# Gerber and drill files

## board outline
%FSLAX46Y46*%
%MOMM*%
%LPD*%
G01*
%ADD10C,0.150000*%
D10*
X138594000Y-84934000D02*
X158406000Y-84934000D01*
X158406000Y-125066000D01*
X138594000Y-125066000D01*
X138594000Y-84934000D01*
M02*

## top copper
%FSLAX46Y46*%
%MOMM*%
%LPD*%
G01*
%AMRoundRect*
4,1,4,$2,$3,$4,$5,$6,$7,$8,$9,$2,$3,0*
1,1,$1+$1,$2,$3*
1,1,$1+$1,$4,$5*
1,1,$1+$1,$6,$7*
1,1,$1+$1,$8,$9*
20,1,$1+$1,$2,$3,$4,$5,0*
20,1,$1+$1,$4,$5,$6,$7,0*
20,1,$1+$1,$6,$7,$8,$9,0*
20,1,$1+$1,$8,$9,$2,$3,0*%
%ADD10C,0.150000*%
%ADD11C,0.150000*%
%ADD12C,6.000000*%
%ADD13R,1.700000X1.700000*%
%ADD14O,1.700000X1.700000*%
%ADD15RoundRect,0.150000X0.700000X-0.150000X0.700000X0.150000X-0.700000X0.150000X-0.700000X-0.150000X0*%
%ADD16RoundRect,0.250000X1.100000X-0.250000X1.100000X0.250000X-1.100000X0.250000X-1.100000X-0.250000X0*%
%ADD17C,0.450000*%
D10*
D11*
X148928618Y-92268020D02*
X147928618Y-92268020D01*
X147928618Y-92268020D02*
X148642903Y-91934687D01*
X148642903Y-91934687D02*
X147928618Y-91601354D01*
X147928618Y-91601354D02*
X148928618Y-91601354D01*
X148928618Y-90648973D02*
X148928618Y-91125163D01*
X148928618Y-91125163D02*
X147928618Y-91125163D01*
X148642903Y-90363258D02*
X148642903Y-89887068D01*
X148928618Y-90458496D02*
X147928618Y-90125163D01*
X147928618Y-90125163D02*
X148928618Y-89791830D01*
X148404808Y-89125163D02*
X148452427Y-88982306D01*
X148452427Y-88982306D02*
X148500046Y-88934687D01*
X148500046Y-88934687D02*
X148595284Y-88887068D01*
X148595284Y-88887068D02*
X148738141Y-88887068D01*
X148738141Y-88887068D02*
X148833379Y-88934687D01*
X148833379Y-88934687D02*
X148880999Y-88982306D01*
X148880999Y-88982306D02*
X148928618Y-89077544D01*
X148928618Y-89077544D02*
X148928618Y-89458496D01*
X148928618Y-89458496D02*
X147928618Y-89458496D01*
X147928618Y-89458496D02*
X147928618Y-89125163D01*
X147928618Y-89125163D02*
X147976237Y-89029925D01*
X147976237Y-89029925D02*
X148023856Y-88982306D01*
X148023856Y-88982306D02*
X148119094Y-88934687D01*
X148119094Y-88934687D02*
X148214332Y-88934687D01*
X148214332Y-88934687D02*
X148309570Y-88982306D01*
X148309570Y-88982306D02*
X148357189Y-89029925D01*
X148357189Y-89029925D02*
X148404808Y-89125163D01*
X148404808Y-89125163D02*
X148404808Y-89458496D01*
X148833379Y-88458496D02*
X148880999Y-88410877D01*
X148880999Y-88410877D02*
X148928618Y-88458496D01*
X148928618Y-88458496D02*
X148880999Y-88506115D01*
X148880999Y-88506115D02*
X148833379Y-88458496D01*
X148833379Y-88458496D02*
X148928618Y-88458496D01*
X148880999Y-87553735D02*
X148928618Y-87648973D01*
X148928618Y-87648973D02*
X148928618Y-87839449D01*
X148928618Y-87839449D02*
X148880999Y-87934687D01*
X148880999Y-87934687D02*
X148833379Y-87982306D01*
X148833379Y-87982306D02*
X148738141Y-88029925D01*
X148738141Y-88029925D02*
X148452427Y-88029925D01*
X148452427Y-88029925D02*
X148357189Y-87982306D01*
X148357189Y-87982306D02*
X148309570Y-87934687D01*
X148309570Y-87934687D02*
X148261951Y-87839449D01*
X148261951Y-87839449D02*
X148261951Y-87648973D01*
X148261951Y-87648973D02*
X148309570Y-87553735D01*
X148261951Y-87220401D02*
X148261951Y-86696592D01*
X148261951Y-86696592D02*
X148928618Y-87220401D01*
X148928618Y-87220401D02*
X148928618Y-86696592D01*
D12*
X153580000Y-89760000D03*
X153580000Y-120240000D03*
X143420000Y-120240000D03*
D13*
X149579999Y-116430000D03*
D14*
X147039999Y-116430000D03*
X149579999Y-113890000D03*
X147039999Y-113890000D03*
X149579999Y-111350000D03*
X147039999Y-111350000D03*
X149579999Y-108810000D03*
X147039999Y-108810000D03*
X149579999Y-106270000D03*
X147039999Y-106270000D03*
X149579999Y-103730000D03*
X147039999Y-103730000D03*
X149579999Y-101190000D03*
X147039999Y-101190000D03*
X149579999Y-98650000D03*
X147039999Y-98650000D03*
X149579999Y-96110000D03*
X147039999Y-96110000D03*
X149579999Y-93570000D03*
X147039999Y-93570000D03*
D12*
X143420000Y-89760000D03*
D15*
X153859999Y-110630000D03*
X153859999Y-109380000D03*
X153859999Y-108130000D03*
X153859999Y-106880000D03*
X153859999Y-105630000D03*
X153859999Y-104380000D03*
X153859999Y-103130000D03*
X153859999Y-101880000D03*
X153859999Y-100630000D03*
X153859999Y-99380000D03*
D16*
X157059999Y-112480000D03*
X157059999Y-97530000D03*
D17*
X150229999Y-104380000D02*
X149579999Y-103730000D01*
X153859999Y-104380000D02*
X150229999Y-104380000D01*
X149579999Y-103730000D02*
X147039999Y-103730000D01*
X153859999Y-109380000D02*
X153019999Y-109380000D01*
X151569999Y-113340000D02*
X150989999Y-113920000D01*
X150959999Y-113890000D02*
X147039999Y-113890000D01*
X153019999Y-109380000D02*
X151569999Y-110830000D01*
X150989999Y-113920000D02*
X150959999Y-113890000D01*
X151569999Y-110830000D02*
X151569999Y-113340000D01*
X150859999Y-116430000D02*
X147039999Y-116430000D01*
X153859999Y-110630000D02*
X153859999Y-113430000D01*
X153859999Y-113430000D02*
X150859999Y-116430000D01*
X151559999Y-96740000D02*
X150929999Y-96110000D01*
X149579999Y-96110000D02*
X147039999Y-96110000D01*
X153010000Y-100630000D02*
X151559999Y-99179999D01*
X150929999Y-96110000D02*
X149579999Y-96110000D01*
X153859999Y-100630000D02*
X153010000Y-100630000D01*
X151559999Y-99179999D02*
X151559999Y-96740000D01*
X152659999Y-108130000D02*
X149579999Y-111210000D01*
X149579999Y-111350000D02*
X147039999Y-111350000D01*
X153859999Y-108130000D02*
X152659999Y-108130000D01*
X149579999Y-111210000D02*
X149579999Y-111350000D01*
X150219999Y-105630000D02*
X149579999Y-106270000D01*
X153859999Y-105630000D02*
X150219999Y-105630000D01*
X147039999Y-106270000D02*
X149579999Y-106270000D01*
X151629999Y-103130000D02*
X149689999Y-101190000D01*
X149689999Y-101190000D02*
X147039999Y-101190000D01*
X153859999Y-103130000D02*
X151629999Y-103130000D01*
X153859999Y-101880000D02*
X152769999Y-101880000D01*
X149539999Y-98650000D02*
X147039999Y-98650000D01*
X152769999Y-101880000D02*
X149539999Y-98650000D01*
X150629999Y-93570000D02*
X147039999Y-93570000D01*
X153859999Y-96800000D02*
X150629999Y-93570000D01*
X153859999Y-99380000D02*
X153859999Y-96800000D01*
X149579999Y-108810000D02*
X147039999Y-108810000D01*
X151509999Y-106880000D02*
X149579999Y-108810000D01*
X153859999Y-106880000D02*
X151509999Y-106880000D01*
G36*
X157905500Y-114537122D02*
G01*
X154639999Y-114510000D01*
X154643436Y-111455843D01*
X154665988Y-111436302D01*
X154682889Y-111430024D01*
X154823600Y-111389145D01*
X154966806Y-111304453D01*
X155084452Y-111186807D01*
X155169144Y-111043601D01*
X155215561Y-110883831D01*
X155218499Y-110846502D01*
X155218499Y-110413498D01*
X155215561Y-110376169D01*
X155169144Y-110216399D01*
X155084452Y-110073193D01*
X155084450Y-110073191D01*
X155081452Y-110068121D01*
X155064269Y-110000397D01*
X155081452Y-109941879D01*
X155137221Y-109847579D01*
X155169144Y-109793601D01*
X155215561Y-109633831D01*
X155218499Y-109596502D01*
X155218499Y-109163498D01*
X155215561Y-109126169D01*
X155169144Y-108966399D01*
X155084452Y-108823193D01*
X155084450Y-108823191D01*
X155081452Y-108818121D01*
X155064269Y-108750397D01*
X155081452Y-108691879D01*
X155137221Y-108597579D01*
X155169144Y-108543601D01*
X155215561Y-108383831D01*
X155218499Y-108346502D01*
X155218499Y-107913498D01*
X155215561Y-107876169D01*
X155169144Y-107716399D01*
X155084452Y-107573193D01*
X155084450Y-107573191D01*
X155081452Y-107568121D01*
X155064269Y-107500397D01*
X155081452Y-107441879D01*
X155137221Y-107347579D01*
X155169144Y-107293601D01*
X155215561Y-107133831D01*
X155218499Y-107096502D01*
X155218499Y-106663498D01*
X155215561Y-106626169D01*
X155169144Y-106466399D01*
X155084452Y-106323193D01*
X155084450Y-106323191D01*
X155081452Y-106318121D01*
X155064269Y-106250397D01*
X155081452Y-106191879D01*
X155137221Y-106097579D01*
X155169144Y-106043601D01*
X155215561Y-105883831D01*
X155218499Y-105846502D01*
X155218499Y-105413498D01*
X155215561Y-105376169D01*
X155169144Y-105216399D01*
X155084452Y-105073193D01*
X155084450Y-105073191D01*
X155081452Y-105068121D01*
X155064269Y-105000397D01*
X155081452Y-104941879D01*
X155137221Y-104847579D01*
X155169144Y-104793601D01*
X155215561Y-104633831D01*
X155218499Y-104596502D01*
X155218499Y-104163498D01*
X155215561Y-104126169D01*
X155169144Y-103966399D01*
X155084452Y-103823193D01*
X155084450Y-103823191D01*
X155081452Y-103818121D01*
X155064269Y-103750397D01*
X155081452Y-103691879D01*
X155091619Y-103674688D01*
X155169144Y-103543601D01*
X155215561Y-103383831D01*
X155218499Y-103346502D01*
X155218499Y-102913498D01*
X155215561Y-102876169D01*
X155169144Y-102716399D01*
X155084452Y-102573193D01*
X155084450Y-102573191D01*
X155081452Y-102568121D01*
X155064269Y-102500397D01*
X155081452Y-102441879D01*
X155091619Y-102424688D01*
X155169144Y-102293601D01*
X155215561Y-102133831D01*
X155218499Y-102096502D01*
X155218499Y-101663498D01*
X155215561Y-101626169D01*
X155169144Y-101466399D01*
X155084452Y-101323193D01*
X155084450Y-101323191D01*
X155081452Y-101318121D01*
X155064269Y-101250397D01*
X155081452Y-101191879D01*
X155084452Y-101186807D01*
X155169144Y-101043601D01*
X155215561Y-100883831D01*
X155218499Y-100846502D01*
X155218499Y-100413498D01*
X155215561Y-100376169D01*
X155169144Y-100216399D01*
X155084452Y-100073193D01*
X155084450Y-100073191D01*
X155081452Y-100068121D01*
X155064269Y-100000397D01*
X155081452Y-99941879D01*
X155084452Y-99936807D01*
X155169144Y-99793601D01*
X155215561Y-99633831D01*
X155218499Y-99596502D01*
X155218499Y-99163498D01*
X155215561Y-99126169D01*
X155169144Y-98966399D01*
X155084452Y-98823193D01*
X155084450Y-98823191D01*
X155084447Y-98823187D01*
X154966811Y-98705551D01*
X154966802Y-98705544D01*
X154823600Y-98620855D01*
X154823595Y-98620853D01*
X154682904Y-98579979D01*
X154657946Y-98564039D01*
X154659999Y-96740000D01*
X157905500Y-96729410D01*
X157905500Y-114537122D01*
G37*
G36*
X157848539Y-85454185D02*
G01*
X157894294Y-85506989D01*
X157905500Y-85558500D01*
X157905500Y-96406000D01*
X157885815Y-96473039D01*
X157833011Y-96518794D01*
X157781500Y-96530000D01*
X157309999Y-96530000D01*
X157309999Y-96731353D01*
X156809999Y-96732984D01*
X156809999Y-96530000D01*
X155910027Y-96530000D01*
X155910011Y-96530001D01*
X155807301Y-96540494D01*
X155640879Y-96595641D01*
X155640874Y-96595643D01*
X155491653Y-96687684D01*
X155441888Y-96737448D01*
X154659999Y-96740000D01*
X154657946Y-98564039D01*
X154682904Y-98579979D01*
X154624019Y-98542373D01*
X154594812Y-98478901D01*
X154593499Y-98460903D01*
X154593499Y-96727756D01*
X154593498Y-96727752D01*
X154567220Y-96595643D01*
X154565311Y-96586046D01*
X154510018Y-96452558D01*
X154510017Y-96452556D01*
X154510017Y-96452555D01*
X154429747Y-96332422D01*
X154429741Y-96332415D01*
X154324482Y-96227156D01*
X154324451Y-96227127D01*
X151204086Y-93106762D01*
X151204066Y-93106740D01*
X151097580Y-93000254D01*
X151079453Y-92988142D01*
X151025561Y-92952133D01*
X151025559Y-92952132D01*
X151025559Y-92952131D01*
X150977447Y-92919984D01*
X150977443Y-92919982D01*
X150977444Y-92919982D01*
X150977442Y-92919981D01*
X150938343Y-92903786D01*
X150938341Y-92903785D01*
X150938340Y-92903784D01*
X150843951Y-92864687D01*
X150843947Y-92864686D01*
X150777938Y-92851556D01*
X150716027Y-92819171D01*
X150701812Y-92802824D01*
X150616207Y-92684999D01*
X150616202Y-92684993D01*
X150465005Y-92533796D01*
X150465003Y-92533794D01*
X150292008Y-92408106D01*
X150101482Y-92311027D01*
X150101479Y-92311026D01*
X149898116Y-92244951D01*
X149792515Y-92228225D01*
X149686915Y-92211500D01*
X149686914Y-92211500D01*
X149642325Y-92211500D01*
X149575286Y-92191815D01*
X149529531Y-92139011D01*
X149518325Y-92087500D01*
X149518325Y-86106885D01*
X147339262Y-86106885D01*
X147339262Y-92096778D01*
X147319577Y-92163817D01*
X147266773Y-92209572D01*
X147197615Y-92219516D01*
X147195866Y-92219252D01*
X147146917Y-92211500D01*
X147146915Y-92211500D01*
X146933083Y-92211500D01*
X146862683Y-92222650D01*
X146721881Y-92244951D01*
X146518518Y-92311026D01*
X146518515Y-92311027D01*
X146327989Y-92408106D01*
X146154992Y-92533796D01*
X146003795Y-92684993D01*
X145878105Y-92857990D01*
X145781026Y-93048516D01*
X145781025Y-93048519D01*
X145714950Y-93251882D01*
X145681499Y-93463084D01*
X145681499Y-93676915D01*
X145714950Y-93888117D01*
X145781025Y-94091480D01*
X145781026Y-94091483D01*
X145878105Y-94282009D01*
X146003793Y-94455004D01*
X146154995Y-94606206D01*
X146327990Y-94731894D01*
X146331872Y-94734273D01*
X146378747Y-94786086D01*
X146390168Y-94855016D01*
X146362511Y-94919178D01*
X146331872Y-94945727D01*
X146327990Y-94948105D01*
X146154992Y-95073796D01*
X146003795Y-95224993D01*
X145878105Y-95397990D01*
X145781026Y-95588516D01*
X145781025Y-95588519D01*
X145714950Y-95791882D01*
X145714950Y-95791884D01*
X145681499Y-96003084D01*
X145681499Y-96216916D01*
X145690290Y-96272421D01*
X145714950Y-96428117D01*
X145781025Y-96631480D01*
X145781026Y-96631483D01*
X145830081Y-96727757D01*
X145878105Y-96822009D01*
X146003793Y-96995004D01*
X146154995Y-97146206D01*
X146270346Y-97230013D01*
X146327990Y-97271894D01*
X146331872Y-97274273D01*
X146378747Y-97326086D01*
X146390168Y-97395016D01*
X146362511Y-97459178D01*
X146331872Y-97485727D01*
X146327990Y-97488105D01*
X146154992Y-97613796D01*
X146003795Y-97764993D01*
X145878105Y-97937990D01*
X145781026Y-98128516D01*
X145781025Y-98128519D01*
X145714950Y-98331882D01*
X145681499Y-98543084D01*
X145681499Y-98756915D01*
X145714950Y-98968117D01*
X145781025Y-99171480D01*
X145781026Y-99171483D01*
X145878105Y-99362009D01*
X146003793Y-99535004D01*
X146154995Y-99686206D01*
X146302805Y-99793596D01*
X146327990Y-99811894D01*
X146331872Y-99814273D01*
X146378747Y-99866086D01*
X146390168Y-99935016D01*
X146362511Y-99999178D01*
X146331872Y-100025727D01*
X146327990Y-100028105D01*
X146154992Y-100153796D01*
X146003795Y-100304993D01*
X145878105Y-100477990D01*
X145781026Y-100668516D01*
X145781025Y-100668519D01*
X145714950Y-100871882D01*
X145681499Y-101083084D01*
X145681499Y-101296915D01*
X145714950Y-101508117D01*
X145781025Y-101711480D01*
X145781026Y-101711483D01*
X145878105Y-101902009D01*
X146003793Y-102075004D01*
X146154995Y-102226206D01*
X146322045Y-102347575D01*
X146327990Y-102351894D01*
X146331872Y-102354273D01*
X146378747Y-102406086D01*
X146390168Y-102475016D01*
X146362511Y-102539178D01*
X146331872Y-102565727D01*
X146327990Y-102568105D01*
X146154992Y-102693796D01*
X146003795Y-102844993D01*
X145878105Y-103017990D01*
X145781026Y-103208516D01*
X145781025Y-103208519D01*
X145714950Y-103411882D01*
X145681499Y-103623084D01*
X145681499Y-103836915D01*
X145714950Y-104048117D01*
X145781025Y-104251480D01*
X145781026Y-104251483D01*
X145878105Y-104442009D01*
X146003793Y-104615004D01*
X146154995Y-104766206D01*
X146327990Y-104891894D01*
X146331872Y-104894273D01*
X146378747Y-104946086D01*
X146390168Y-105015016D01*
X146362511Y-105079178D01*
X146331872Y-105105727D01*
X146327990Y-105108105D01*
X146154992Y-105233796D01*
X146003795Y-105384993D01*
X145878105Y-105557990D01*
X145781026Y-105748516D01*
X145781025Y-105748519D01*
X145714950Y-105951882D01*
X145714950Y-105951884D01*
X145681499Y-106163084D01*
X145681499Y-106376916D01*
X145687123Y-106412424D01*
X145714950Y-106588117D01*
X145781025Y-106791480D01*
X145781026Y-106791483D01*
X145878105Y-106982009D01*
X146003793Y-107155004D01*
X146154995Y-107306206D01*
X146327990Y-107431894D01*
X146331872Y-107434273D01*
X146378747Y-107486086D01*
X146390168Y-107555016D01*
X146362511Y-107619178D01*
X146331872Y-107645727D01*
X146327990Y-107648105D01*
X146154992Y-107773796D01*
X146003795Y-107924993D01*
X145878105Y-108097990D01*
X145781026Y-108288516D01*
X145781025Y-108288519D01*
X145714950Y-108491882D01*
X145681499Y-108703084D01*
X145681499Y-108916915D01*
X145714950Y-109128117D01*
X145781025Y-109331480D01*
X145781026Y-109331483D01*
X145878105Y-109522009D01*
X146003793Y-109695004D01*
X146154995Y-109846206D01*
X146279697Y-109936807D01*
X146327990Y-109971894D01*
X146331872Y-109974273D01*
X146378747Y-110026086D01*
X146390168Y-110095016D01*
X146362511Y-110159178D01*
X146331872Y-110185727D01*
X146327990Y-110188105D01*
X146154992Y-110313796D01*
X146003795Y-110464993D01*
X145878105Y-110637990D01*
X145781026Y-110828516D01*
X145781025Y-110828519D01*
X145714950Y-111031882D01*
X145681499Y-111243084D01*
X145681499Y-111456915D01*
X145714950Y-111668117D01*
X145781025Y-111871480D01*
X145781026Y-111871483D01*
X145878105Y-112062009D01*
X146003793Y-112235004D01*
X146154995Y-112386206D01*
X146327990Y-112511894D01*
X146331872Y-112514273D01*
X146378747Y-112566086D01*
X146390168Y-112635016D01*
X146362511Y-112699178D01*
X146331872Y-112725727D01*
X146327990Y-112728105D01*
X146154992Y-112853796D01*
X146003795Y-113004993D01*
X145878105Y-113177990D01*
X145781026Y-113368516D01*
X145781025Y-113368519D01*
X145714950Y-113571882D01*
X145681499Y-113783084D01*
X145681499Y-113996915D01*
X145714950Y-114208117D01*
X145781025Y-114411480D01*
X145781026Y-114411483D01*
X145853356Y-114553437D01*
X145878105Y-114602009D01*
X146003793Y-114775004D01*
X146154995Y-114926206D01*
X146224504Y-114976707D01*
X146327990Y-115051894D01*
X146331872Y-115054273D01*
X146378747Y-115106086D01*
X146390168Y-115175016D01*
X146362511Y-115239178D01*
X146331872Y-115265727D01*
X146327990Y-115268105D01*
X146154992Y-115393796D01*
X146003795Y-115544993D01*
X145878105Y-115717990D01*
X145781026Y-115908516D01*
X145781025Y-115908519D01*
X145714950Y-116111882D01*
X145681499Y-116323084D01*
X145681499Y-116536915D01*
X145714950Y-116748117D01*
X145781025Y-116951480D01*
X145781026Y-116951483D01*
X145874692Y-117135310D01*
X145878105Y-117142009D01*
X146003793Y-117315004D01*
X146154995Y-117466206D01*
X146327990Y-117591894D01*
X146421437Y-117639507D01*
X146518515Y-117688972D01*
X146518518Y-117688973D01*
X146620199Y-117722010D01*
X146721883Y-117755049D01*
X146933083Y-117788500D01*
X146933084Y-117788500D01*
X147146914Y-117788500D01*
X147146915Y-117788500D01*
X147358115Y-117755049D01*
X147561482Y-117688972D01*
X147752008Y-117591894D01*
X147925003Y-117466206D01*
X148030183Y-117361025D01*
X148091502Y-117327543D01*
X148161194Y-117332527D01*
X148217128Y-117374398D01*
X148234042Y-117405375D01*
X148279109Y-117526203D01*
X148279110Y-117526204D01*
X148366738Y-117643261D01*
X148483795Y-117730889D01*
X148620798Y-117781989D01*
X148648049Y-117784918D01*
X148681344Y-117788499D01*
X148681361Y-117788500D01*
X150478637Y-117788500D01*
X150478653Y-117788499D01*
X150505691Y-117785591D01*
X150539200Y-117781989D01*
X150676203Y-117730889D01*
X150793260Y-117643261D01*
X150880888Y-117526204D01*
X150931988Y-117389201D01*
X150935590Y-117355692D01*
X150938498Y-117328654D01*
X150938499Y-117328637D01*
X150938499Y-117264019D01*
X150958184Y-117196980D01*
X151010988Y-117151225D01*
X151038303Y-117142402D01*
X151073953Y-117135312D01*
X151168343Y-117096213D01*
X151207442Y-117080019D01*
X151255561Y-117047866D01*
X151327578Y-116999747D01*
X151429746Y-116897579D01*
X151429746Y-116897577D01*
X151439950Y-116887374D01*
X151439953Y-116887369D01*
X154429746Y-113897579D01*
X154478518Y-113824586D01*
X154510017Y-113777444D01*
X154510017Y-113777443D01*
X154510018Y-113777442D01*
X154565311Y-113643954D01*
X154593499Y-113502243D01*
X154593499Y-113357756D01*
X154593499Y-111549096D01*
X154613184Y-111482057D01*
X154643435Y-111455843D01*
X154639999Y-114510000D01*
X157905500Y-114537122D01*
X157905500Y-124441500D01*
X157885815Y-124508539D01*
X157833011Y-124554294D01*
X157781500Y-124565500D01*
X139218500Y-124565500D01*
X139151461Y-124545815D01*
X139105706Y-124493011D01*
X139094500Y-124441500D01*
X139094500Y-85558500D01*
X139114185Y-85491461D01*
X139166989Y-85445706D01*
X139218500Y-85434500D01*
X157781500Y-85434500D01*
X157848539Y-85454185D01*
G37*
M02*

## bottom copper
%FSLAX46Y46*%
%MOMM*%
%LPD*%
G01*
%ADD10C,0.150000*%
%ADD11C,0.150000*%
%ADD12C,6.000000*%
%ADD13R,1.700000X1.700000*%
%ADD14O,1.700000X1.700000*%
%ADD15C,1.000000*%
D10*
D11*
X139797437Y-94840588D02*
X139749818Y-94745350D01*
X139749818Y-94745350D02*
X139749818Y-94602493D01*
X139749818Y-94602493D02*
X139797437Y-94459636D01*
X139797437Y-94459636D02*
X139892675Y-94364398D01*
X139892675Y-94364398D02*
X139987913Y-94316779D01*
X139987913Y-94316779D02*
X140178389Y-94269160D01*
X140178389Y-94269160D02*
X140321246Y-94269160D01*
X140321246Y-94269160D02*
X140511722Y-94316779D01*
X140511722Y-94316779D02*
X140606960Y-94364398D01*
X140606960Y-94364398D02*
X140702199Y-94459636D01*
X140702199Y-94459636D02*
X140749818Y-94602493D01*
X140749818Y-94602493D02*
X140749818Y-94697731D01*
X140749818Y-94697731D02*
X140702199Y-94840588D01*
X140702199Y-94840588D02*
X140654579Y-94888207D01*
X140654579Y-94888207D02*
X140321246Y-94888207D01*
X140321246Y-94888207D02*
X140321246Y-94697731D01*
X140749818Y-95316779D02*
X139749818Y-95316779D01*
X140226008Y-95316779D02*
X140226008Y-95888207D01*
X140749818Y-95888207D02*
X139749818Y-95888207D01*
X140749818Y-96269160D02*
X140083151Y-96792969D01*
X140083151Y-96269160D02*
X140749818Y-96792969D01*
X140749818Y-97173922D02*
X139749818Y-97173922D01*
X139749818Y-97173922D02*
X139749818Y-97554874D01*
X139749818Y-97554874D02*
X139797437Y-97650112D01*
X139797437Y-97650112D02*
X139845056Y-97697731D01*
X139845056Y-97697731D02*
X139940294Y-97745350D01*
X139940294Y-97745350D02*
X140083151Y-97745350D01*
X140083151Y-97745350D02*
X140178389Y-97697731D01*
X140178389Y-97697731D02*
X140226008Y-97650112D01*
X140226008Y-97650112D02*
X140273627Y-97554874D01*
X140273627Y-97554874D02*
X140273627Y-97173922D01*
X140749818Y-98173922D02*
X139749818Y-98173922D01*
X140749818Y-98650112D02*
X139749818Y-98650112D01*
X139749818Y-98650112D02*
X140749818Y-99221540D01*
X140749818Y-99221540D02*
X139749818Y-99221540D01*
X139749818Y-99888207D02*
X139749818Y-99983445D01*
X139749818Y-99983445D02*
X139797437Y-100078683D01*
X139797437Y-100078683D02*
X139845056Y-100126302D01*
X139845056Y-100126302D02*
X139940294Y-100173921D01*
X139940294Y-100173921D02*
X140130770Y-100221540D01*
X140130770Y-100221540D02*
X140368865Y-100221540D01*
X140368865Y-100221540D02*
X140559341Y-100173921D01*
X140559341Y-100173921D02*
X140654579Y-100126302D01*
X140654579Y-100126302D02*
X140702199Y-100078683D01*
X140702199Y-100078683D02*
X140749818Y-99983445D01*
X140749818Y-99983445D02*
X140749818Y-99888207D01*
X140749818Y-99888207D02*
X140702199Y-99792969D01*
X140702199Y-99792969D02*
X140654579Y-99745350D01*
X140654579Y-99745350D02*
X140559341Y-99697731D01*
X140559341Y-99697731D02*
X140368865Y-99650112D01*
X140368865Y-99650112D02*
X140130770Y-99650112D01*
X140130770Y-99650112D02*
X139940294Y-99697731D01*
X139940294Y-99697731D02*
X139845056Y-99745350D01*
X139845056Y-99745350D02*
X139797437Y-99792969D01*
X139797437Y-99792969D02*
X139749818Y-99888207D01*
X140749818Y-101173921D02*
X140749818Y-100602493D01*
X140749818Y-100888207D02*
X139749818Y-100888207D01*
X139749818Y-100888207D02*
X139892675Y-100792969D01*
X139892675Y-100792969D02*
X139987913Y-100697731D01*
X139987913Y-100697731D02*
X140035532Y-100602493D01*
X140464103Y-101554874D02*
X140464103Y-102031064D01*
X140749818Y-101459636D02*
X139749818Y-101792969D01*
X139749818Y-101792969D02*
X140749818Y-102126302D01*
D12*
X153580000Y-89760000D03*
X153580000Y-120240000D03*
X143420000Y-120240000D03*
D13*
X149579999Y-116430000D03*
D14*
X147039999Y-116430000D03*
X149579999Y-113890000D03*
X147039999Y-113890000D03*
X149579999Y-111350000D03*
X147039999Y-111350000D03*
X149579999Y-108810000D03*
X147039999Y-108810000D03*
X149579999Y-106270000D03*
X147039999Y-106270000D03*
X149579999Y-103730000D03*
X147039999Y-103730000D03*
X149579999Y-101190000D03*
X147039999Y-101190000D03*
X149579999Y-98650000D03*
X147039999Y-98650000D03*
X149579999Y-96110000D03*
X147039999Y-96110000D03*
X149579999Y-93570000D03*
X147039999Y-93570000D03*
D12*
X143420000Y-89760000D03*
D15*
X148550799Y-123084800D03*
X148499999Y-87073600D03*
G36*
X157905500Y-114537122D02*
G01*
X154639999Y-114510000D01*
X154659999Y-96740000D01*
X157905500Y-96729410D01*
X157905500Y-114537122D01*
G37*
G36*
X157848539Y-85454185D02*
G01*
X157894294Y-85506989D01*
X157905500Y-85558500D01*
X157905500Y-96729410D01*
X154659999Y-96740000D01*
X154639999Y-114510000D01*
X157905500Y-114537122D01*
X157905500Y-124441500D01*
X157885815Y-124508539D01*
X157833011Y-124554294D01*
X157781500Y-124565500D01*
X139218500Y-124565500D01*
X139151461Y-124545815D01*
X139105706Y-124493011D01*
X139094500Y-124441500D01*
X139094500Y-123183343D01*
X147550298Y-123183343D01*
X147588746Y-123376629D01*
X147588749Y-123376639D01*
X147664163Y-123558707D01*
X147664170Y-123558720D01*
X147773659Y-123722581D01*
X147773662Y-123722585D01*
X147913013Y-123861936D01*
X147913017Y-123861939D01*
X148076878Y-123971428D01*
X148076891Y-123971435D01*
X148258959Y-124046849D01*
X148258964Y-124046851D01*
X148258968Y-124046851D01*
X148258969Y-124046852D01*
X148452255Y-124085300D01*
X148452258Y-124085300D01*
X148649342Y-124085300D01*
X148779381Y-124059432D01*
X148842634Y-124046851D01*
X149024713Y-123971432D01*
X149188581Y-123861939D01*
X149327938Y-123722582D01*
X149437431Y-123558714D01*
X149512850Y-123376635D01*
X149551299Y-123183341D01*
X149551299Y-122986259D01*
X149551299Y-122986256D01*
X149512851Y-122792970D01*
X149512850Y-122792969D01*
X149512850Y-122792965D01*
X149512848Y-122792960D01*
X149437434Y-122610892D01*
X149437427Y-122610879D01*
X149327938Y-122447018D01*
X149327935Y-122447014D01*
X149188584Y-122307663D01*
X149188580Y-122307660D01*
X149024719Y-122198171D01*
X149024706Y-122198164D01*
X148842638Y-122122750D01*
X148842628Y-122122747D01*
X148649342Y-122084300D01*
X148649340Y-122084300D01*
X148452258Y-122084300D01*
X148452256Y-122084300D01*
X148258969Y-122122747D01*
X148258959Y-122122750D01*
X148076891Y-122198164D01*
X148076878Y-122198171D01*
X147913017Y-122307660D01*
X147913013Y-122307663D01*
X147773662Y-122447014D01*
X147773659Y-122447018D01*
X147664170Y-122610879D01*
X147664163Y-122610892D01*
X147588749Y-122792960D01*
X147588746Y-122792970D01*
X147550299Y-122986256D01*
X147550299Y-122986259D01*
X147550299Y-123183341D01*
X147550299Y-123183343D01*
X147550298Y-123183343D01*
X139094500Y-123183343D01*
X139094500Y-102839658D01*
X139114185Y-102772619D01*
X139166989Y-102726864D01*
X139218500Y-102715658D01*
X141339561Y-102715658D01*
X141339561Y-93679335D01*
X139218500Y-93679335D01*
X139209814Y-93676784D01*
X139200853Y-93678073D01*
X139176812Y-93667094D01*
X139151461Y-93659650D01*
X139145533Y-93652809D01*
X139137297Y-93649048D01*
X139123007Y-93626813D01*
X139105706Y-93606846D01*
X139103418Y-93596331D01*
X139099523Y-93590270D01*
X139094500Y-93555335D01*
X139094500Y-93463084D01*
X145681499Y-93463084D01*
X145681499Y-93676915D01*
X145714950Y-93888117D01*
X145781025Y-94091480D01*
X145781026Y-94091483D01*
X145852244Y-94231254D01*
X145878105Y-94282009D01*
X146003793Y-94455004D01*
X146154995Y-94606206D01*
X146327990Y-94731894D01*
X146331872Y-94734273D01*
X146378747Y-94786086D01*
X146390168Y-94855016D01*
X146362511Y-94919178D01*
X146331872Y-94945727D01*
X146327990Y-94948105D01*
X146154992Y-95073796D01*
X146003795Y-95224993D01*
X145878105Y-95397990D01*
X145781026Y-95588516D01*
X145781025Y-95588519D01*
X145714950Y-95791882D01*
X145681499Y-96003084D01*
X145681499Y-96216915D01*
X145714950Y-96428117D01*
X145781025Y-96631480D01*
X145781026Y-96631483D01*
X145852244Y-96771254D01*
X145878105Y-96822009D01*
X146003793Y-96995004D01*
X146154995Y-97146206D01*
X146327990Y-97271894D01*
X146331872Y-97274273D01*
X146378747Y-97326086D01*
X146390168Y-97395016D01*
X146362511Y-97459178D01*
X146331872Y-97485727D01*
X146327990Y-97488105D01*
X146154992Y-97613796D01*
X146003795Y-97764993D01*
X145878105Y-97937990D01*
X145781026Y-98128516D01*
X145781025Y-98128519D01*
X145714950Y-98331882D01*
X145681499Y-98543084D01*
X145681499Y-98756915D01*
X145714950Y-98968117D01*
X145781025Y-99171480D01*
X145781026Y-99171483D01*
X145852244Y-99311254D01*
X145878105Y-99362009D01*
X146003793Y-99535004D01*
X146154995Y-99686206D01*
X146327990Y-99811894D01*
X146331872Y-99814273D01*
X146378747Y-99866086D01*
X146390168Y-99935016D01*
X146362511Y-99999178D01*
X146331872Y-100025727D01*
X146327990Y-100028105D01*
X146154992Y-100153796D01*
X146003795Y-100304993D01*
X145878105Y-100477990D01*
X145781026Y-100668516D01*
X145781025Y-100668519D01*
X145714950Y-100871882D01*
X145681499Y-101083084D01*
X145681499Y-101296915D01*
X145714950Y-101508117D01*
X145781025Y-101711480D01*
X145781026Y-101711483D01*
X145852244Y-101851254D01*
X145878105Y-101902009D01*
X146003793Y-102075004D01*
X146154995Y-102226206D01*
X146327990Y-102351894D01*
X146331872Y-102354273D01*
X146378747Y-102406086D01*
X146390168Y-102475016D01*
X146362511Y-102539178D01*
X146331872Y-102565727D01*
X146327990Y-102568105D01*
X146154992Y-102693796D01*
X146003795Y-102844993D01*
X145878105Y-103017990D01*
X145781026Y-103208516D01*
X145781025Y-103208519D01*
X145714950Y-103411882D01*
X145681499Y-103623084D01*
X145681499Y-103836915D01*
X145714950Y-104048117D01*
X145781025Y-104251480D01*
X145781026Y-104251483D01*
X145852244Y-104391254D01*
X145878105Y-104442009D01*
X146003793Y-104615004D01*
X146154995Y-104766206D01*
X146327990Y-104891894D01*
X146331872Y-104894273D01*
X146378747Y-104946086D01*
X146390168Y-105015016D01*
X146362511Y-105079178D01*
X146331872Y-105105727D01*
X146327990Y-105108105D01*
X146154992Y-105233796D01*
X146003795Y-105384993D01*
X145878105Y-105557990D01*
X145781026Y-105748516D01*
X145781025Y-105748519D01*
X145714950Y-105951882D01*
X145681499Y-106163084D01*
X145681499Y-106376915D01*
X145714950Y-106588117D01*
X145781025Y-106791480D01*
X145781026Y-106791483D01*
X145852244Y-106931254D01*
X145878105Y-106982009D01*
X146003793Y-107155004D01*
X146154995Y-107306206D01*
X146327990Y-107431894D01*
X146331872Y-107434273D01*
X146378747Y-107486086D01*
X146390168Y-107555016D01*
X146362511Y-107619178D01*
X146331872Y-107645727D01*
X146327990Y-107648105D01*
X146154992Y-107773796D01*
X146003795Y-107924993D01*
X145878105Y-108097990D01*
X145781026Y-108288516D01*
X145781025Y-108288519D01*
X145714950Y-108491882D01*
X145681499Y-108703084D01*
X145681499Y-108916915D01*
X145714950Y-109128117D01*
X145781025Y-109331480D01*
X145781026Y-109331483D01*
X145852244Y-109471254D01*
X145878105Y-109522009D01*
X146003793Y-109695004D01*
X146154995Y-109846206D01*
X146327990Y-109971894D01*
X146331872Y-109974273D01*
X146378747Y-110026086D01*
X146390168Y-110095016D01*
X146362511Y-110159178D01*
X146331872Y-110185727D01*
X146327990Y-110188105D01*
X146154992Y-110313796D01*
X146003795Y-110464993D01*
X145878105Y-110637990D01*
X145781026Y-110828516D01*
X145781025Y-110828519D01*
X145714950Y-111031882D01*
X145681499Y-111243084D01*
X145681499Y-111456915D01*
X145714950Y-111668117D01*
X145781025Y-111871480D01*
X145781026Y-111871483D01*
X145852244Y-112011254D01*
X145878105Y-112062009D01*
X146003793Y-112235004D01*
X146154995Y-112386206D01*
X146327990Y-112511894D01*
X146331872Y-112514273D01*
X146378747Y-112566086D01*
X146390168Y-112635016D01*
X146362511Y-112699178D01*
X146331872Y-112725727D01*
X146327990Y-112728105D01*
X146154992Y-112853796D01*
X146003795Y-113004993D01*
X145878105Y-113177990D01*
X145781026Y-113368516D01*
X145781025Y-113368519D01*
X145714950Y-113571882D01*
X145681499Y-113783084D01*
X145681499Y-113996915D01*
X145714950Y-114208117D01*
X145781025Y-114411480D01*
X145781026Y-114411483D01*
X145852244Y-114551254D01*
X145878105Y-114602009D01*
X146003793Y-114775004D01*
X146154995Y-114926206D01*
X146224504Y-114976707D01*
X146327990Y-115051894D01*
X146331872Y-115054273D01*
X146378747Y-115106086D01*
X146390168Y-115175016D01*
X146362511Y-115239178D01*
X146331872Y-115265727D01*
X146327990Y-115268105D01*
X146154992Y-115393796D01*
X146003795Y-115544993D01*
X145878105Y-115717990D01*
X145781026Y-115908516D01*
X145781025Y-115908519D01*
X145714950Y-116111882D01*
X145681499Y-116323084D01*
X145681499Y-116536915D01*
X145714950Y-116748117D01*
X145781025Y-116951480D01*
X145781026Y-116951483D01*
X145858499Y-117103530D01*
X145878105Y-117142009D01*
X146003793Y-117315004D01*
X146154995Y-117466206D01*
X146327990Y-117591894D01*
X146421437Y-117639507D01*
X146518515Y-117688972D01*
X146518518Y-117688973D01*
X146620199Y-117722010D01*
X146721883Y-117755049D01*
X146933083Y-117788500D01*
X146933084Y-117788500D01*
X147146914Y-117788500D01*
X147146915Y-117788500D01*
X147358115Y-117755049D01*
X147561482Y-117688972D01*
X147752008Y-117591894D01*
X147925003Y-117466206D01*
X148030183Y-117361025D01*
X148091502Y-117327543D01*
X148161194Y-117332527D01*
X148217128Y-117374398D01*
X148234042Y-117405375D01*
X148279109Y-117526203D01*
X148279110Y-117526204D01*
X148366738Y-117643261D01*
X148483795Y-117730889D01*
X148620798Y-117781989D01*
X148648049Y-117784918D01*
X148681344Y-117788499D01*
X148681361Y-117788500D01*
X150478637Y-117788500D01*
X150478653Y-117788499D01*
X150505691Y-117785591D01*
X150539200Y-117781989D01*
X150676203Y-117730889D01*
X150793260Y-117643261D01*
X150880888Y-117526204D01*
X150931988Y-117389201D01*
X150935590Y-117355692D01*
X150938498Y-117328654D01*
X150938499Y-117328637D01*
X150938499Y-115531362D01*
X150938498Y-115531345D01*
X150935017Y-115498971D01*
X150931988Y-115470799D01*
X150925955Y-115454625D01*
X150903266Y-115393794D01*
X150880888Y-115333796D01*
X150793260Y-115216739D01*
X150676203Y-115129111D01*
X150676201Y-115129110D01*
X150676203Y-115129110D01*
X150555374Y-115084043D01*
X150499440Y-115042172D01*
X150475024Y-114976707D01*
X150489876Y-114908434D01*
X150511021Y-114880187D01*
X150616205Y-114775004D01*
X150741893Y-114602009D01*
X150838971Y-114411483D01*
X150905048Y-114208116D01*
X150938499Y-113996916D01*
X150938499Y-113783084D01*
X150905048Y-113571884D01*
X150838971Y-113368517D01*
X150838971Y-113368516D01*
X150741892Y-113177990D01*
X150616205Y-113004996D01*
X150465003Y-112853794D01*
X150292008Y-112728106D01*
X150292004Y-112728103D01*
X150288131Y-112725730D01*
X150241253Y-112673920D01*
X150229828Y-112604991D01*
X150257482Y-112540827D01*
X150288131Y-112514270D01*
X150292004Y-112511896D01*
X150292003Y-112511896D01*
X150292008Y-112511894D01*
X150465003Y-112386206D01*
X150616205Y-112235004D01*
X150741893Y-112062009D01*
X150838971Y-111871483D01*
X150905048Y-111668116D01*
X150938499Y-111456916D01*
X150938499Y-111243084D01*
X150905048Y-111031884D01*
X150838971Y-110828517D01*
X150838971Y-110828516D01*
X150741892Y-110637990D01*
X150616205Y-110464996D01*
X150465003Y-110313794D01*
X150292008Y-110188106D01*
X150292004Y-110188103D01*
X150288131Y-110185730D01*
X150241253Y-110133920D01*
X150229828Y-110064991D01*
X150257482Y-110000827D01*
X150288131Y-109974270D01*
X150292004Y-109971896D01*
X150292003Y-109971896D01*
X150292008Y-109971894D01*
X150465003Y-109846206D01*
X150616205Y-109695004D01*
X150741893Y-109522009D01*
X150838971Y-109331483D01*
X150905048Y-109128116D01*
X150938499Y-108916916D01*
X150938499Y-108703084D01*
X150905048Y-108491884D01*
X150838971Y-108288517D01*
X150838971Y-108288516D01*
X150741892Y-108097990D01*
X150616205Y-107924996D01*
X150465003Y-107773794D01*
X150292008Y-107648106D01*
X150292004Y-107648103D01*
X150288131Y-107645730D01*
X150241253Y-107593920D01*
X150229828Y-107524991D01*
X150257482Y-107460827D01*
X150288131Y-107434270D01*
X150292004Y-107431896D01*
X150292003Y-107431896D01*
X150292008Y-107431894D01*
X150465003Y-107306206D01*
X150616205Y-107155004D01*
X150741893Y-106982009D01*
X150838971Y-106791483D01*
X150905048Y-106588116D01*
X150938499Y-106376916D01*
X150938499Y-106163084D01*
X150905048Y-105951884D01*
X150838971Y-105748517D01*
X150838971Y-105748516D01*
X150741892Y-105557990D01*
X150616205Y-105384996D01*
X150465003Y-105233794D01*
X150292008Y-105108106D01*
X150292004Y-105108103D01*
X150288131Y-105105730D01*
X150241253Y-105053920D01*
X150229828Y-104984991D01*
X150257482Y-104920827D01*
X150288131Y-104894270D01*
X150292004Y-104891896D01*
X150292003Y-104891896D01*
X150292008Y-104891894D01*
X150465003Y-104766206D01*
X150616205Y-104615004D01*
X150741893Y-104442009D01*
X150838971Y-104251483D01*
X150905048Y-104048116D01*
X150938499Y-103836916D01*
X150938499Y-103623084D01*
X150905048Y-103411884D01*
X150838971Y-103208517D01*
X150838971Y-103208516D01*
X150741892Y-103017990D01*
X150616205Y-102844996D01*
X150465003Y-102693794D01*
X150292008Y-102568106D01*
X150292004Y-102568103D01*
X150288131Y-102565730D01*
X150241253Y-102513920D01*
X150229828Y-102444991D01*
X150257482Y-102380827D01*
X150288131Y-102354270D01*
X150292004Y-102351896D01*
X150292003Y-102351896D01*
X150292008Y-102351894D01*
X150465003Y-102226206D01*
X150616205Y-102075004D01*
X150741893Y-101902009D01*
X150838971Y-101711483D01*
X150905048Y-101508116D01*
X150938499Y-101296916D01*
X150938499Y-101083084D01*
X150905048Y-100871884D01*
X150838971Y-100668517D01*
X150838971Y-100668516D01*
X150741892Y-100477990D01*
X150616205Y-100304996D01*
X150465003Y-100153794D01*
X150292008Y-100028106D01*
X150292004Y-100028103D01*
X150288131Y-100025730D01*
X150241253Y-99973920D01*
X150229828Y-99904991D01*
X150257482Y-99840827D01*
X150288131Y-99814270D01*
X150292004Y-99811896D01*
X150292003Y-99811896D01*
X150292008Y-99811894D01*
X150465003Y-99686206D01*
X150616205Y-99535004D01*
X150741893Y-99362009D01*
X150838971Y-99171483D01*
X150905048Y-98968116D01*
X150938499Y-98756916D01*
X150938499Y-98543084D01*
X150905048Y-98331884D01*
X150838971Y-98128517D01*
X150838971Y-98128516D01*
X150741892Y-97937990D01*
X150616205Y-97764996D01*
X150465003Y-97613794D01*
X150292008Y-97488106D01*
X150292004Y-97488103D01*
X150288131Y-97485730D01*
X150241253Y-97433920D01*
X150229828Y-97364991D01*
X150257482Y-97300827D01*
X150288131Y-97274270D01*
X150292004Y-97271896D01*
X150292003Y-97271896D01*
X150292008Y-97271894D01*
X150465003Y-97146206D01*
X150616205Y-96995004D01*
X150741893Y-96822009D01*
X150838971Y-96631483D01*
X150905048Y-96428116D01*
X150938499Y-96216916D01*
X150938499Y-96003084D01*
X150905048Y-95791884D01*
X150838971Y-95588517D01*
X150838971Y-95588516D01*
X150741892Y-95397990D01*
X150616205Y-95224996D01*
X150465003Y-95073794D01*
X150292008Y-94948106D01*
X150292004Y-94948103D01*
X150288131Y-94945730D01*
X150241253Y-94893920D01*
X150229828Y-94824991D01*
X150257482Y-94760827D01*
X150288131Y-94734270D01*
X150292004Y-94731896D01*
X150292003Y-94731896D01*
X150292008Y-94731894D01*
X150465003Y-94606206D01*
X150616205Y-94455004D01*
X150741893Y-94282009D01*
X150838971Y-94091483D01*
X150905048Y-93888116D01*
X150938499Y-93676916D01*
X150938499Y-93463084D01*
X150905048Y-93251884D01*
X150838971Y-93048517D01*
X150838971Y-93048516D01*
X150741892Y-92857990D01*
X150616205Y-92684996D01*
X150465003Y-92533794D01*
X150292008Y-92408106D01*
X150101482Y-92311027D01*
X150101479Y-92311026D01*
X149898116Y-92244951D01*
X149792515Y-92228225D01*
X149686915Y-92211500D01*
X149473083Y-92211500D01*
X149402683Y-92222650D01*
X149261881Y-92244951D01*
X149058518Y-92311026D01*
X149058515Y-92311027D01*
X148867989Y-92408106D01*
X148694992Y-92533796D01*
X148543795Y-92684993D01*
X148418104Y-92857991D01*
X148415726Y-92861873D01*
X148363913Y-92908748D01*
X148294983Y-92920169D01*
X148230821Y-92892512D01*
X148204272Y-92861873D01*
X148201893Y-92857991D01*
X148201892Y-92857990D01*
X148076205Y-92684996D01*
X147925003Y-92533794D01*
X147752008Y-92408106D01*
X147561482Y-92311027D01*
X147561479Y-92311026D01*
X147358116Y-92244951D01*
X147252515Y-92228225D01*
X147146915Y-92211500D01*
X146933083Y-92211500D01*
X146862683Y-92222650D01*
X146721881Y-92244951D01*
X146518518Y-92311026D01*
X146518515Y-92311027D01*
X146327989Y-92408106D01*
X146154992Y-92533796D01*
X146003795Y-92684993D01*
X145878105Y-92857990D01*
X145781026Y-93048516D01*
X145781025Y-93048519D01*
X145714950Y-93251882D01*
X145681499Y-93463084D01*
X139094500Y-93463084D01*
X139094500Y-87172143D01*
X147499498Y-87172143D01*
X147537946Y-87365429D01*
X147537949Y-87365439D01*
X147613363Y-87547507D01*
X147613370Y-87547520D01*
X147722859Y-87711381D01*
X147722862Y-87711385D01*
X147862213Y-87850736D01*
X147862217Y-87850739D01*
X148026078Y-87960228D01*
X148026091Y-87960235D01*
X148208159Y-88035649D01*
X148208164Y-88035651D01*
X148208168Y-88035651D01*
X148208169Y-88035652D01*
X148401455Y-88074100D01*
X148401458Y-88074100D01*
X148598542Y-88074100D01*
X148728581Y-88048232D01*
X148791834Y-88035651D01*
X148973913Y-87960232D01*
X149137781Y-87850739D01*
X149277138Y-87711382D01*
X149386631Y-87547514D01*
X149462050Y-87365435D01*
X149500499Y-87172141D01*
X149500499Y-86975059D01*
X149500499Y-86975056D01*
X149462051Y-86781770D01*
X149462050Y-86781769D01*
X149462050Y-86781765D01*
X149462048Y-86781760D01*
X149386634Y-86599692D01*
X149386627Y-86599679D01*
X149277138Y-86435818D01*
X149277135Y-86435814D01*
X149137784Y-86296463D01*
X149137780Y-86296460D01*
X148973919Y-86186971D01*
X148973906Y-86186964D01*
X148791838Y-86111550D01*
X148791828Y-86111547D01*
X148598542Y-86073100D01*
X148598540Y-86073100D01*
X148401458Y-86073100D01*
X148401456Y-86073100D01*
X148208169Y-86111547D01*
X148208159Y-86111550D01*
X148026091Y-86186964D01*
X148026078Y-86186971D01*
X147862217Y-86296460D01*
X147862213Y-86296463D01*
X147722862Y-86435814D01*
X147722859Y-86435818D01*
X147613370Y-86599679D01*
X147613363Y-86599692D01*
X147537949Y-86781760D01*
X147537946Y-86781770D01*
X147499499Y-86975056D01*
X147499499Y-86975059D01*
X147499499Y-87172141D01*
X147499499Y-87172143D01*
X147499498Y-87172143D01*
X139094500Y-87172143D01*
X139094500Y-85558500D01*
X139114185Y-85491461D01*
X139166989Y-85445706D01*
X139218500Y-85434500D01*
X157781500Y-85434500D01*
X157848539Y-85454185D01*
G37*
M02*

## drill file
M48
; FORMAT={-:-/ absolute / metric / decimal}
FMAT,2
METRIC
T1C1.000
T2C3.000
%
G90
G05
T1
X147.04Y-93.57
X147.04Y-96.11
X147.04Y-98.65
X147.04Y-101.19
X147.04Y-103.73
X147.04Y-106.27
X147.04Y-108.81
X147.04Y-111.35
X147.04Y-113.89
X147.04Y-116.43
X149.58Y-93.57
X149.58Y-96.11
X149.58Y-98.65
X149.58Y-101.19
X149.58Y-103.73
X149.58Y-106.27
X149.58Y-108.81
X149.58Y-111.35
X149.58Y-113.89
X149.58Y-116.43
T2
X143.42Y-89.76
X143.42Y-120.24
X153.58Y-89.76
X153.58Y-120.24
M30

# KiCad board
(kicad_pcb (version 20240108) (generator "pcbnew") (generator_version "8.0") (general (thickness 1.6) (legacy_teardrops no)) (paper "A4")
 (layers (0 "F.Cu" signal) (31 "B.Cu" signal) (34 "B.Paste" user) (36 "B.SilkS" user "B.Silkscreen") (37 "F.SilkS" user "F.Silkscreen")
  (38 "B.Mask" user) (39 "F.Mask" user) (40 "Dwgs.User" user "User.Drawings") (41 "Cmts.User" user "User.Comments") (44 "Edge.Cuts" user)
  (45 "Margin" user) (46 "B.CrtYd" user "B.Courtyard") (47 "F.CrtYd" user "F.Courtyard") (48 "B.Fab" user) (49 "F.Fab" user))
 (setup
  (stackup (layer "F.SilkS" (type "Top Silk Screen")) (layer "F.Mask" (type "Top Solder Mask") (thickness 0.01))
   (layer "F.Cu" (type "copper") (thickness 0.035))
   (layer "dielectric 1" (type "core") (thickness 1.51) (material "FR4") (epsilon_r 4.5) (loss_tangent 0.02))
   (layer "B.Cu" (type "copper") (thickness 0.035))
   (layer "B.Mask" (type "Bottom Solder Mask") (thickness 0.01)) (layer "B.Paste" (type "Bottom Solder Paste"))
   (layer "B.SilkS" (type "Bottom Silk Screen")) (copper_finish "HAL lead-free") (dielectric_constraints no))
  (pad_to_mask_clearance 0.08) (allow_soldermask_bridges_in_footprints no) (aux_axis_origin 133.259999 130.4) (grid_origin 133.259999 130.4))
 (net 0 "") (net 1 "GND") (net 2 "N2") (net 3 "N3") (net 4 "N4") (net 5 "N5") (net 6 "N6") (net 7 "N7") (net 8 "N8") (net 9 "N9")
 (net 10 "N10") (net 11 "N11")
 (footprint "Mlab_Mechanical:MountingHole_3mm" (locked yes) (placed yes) (layer "F.Cu") (at 153.58 89.76)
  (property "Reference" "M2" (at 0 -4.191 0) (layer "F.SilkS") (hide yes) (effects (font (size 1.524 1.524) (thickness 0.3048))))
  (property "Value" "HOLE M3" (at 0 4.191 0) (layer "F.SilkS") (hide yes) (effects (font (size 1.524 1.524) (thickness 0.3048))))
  (pad "1" thru_hole circle (at 0 0) (size 6 6) (drill 3) (layers "*.Cu" "*.Mask") (remove_unused_layers no) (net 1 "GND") (clearance 1)
   (zone_connect 2)))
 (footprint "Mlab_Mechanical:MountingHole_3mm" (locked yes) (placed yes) (layer "F.Cu") (at 153.58 120.24)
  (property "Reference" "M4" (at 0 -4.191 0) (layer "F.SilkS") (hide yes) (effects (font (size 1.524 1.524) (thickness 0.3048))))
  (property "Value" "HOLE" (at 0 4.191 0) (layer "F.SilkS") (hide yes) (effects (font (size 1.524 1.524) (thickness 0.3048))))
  (pad "1" thru_hole circle (at 0 0) (size 6 6) (drill 3) (layers "*.Cu" "*.Mask") (remove_unused_layers no) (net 1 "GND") (clearance 1)
   (zone_connect 2)))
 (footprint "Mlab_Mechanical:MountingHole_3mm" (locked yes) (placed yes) (layer "F.Cu") (at 143.42 120.24)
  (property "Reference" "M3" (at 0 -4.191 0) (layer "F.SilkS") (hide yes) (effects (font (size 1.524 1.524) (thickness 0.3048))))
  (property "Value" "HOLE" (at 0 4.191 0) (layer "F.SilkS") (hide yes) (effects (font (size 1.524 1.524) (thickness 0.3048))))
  (pad "1" thru_hole circle (at 0 0) (size 6 6) (drill 3) (layers "*.Cu" "*.Mask") (remove_unused_layers no) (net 1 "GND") (clearance 1)
   (zone_connect 2)))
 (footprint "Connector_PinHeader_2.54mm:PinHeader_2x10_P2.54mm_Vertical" (layer "F.Cu") (at 149.579999 116.43 180)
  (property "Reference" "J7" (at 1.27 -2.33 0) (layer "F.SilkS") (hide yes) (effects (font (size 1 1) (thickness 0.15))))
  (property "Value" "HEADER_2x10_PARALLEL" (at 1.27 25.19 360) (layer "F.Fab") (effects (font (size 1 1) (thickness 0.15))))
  (pad "1" thru_hole rect (at 0 0 180) (size 1.7 1.7) (drill 1) (layers "*.Cu" "*.Mask") (remove_unused_layers no) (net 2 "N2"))
  (pad "2" thru_hole oval (at 2.54 0 180) (size 1.7 1.7) (drill 1) (layers "*.Cu" "*.Mask") (remove_unused_layers no) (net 2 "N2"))
  (pad "3" thru_hole oval (at 0 2.54 180) (size 1.7 1.7) (drill 1) (layers "*.Cu" "*.Mask") (remove_unused_layers no) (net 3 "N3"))
  (pad "4" thru_hole oval (at 2.54 2.54 180) (size 1.7 1.7) (drill 1) (layers "*.Cu" "*.Mask") (remove_unused_layers no) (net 3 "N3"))
  (pad "5" thru_hole oval (at 0 5.08 180) (size 1.7 1.7) (drill 1) (layers "*.Cu" "*.Mask") (remove_unused_layers no) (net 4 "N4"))
  (pad "6" thru_hole oval (at 2.54 5.08 180) (size 1.7 1.7) (drill 1) (layers "*.Cu" "*.Mask") (remove_unused_layers no) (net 4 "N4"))
  (pad "7" thru_hole oval (at 0 7.62 180) (size 1.7 1.7) (drill 1) (layers "*.Cu" "*.Mask") (remove_unused_layers no) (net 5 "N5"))
  (pad "8" thru_hole oval (at 2.54 7.62 180) (size 1.7 1.7) (drill 1) (layers "*.Cu" "*.Mask") (remove_unused_layers no) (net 5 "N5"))
  (pad "9" thru_hole oval (at 0 10.16 180) (size 1.7 1.7) (drill 1) (layers "*.Cu" "*.Mask") (remove_unused_layers no) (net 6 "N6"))
  (pad "10" thru_hole oval (at 2.54 10.16 180) (size 1.7 1.7) (drill 1) (layers "*.Cu" "*.Mask") (remove_unused_layers no) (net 6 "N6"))
  (pad "11" thru_hole oval (at 0 12.7 180) (size 1.7 1.7) (drill 1) (layers "*.Cu" "*.Mask") (remove_unused_layers no) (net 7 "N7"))
  (pad "12" thru_hole oval (at 2.54 12.7 180) (size 1.7 1.7) (drill 1) (layers "*.Cu" "*.Mask") (remove_unused_layers no) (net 7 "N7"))
  (pad "13" thru_hole oval (at 0 15.24 180) (size 1.7 1.7) (drill 1) (layers "*.Cu" "*.Mask") (remove_unused_layers no) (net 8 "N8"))
  (pad "14" thru_hole oval (at 2.54 15.24 180) (size 1.7 1.7) (drill 1) (layers "*.Cu" "*.Mask") (remove_unused_layers no) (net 8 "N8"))
  (pad "15" thru_hole oval (at 0 17.78 180) (size 1.7 1.7) (drill 1) (layers "*.Cu" "*.Mask") (remove_unused_layers no) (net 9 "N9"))
  (pad "16" thru_hole oval (at 2.54 17.78 180) (size 1.7 1.7) (drill 1) (layers "*.Cu" "*.Mask") (remove_unused_layers no) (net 9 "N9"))
  (pad "17" thru_hole oval (at 0 20.32 180) (size 1.7 1.7) (drill 1) (layers "*.Cu" "*.Mask") (remove_unused_layers no) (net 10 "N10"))
  (pad "18" thru_hole oval (at 2.54 20.32 180) (size 1.7 1.7) (drill 1) (layers "*.Cu" "*.Mask") (remove_unused_layers no) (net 10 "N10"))
  (pad "19" thru_hole oval (at 0 22.86 180) (size 1.7 1.7) (drill 1) (layers "*.Cu" "*.Mask") (remove_unused_layers no) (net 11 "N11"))
  (pad "20" thru_hole oval (at 2.54 22.86 180) (size 1.7 1.7) (drill 1) (layers "*.Cu" "*.Mask") (remove_unused_layers no) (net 11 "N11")))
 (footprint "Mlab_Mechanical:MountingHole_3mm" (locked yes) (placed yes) (layer "F.Cu") (at 143.42 89.76)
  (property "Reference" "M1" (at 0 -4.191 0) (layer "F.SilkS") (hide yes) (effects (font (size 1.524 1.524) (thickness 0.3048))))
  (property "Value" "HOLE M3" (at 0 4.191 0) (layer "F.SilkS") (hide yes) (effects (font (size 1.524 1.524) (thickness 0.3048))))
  (pad "1" thru_hole circle (at 0 0) (size 6 6) (drill 3) (layers "*.Cu" "*.Mask") (remove_unused_layers no) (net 1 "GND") (clearance 1)
   (zone_connect 2)))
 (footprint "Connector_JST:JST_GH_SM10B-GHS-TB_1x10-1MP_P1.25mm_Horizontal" (layer "F.Cu") (at 155.709999 105.005 90)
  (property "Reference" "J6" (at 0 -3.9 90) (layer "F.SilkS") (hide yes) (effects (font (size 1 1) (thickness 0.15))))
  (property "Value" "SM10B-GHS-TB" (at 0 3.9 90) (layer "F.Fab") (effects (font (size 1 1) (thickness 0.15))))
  (pad "1" smd roundrect (at -5.625 -1.85 90) (size 0.6 1.7) (layers "F.Cu" "F.Paste" "F.Mask") (roundrect_rratio 0.25) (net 2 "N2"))
  (pad "2" smd roundrect (at -4.375 -1.85 90) (size 0.6 1.7) (layers "F.Cu" "F.Paste" "F.Mask") (roundrect_rratio 0.25) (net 3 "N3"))
  (pad "3" smd roundrect (at -3.125 -1.85 90) (size 0.6 1.7) (layers "F.Cu" "F.Paste" "F.Mask") (roundrect_rratio 0.25) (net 4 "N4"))
  (pad "4" smd roundrect (at -1.875 -1.85 90) (size 0.6 1.7) (layers "F.Cu" "F.Paste" "F.Mask") (roundrect_rratio 0.25) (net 5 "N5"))
  (pad "5" smd roundrect (at -0.625 -1.85 90) (size 0.6 1.7) (layers "F.Cu" "F.Paste" "F.Mask") (roundrect_rratio 0.25) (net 6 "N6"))
  (pad "6" smd roundrect (at 0.625 -1.85 90) (size 0.6 1.7) (layers "F.Cu" "F.Paste" "F.Mask") (roundrect_rratio 0.25) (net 7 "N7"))
  (pad "7" smd roundrect (at 1.875 -1.85 90) (size 0.6 1.7) (layers "F.Cu" "F.Paste" "F.Mask") (roundrect_rratio 0.25) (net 8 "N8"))
  (pad "8" smd roundrect (at 3.125 -1.85 90) (size 0.6 1.7) (layers "F.Cu" "F.Paste" "F.Mask") (roundrect_rratio 0.25) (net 9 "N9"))
  (pad "9" smd roundrect (at 4.375 -1.85 90) (size 0.6 1.7) (layers "F.Cu" "F.Paste" "F.Mask") (roundrect_rratio 0.25) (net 10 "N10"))
  (pad "10" smd roundrect (at 5.625 -1.85 90) (size 0.6 1.7) (layers "F.Cu" "F.Paste" "F.Mask") (roundrect_rratio 0.25) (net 11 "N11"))
  (pad "MP" smd roundrect (at -7.475 1.35 90) (size 1 2.7) (layers "F.Cu" "F.Paste" "F.Mask") (roundrect_rratio 0.25) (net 1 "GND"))
  (pad "MP" smd roundrect (at 7.475 1.35 90) (size 1 2.7) (layers "F.Cu" "F.Paste" "F.Mask") (roundrect_rratio 0.25) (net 1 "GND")))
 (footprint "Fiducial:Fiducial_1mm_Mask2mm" (layer "B.Cu") (at 148.550799 123.0848 180)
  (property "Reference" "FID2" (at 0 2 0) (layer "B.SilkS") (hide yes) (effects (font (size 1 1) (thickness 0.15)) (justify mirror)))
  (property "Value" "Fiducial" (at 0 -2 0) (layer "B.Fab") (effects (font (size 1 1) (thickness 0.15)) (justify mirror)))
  (pad "" smd circle (at 0 0 180) (size 1 1) (layers "B.Cu" "B.Mask") (solder_mask_margin 0.5) (clearance 0.5)))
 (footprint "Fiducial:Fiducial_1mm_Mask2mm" (layer "B.Cu") (at 148.499999 87.0736 180)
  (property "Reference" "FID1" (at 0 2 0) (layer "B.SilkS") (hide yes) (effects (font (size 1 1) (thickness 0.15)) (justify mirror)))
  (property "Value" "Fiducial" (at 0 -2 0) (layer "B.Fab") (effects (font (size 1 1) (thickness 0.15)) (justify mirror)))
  (pad "" smd circle (at 0 0 180) (size 1 1) (layers "B.Cu" "B.Mask") (solder_mask_margin 0.5) (clearance 0.5)))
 (gr_rect (start 138.594 84.934) (end 158.406 125.066) (stroke (width 0.15) (type default)) (fill none) (layer "Edge.Cuts"))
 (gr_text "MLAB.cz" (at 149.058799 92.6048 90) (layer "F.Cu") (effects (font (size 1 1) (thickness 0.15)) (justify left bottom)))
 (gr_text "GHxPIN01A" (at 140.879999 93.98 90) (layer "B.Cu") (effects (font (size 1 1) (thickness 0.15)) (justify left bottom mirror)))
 (segment (start 150.229999 104.38) (end 149.579999 103.73) (width 0.45) (layer "F.Cu") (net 7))
 (segment (start 153.859999 104.38) (end 150.229999 104.38) (width 0.45) (layer "F.Cu") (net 7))
 (segment (start 149.579999 103.73) (end 147.039999 103.73) (width 0.45) (layer "F.Cu") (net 7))
 (segment (start 153.859999 109.38) (end 153.019999 109.38) (width 0.45) (layer "F.Cu") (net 3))
 (segment (start 151.569999 113.34) (end 150.989999 113.92) (width 0.45) (layer "F.Cu") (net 3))
 (segment (start 150.959999 113.89) (end 147.039999 113.89) (width 0.45) (layer "F.Cu") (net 3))
 (segment (start 153.019999 109.38) (end 151.569999 110.83) (width 0.45) (layer "F.Cu") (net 3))
 (segment (start 150.989999 113.92) (end 150.959999 113.89) (width 0.45) (layer "F.Cu") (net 3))
 (segment (start 151.569999 110.83) (end 151.569999 113.34) (width 0.45) (layer "F.Cu") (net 3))
 (segment (start 150.859999 116.43) (end 147.039999 116.43) (width 0.45) (layer "F.Cu") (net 2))
 (segment (start 153.859999 110.63) (end 153.859999 113.43) (width 0.45) (layer "F.Cu") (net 2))
 (segment (start 153.859999 113.43) (end 150.859999 116.43) (width 0.45) (layer "F.Cu") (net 2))
 (segment (start 151.559999 96.74) (end 150.929999 96.11) (width 0.45) (layer "F.Cu") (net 10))
 (segment (start 149.579999 96.11) (end 147.039999 96.11) (width 0.45) (layer "F.Cu") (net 10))
 (segment (start 153.01 100.63) (end 151.559999 99.179999) (width 0.45) (layer "F.Cu") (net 10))
 (segment (start 150.929999 96.11) (end 149.579999 96.11) (width 0.45) (layer "F.Cu") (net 10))
 (segment (start 153.859999 100.63) (end 153.01 100.63) (width 0.45) (layer "F.Cu") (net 10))
 (segment (start 151.559999 99.179999) (end 151.559999 96.74) (width 0.45) (layer "F.Cu") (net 10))
 (segment (start 152.659999 108.13) (end 149.579999 111.21) (width 0.45) (layer "F.Cu") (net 4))
 (segment (start 149.579999 111.35) (end 147.039999 111.35) (width 0.45) (layer "F.Cu") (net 4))
 (segment (start 153.859999 108.13) (end 152.659999 108.13) (width 0.45) (layer "F.Cu") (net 4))
 (segment (start 149.579999 111.21) (end 149.579999 111.35) (width 0.45) (layer "F.Cu") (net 4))
 (segment (start 150.219999 105.63) (end 149.579999 106.27) (width 0.45) (layer "F.Cu") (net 6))
 (segment (start 153.859999 105.63) (end 150.219999 105.63) (width 0.45) (layer "F.Cu") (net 6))
 (segment (start 147.039999 106.27) (end 149.579999 106.27) (width 0.45) (layer "F.Cu") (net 6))
 (segment (start 151.629999 103.13) (end 149.689999 101.19) (width 0.45) (layer "F.Cu") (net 8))
 (segment (start 149.689999 101.19) (end 147.039999 101.19) (width 0.45) (layer "F.Cu") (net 8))
 (segment (start 153.859999 103.13) (end 151.629999 103.13) (width 0.45) (layer "F.Cu") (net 8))
 (segment (start 153.859999 101.88) (end 152.769999 101.88) (width 0.45) (layer "F.Cu") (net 9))
 (segment (start 149.539999 98.65) (end 147.039999 98.65) (width 0.45) (layer "F.Cu") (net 9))
 (segment (start 152.769999 101.88) (end 149.539999 98.65) (width 0.45) (layer "F.Cu") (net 9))
 (segment (start 150.629999 93.57) (end 147.039999 93.57) (width 0.45) (layer "F.Cu") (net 11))
 (segment (start 153.859999 96.8) (end 150.629999 93.57) (width 0.45) (layer "F.Cu") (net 11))
 (segment (start 153.859999 99.38) (end 153.859999 96.8) (width 0.45) (layer "F.Cu") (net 11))
 (segment (start 149.579999 108.81) (end 147.039999 108.81) (width 0.45) (layer "F.Cu") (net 5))
 (segment (start 151.509999 106.88) (end 149.579999 108.81) (width 0.45) (layer "F.Cu") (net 5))
 (segment (start 153.859999 106.88) (end 151.509999 106.88) (width 0.45) (layer "F.Cu") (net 5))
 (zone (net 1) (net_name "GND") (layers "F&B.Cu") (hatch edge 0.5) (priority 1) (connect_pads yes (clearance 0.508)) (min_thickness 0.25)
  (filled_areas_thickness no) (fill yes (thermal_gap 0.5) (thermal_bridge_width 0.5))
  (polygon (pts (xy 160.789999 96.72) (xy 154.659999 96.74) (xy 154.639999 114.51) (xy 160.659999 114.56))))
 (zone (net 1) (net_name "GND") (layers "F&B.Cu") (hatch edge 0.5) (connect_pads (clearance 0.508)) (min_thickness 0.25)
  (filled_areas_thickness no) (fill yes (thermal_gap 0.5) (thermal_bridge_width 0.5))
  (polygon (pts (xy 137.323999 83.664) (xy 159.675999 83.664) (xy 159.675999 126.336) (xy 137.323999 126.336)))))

